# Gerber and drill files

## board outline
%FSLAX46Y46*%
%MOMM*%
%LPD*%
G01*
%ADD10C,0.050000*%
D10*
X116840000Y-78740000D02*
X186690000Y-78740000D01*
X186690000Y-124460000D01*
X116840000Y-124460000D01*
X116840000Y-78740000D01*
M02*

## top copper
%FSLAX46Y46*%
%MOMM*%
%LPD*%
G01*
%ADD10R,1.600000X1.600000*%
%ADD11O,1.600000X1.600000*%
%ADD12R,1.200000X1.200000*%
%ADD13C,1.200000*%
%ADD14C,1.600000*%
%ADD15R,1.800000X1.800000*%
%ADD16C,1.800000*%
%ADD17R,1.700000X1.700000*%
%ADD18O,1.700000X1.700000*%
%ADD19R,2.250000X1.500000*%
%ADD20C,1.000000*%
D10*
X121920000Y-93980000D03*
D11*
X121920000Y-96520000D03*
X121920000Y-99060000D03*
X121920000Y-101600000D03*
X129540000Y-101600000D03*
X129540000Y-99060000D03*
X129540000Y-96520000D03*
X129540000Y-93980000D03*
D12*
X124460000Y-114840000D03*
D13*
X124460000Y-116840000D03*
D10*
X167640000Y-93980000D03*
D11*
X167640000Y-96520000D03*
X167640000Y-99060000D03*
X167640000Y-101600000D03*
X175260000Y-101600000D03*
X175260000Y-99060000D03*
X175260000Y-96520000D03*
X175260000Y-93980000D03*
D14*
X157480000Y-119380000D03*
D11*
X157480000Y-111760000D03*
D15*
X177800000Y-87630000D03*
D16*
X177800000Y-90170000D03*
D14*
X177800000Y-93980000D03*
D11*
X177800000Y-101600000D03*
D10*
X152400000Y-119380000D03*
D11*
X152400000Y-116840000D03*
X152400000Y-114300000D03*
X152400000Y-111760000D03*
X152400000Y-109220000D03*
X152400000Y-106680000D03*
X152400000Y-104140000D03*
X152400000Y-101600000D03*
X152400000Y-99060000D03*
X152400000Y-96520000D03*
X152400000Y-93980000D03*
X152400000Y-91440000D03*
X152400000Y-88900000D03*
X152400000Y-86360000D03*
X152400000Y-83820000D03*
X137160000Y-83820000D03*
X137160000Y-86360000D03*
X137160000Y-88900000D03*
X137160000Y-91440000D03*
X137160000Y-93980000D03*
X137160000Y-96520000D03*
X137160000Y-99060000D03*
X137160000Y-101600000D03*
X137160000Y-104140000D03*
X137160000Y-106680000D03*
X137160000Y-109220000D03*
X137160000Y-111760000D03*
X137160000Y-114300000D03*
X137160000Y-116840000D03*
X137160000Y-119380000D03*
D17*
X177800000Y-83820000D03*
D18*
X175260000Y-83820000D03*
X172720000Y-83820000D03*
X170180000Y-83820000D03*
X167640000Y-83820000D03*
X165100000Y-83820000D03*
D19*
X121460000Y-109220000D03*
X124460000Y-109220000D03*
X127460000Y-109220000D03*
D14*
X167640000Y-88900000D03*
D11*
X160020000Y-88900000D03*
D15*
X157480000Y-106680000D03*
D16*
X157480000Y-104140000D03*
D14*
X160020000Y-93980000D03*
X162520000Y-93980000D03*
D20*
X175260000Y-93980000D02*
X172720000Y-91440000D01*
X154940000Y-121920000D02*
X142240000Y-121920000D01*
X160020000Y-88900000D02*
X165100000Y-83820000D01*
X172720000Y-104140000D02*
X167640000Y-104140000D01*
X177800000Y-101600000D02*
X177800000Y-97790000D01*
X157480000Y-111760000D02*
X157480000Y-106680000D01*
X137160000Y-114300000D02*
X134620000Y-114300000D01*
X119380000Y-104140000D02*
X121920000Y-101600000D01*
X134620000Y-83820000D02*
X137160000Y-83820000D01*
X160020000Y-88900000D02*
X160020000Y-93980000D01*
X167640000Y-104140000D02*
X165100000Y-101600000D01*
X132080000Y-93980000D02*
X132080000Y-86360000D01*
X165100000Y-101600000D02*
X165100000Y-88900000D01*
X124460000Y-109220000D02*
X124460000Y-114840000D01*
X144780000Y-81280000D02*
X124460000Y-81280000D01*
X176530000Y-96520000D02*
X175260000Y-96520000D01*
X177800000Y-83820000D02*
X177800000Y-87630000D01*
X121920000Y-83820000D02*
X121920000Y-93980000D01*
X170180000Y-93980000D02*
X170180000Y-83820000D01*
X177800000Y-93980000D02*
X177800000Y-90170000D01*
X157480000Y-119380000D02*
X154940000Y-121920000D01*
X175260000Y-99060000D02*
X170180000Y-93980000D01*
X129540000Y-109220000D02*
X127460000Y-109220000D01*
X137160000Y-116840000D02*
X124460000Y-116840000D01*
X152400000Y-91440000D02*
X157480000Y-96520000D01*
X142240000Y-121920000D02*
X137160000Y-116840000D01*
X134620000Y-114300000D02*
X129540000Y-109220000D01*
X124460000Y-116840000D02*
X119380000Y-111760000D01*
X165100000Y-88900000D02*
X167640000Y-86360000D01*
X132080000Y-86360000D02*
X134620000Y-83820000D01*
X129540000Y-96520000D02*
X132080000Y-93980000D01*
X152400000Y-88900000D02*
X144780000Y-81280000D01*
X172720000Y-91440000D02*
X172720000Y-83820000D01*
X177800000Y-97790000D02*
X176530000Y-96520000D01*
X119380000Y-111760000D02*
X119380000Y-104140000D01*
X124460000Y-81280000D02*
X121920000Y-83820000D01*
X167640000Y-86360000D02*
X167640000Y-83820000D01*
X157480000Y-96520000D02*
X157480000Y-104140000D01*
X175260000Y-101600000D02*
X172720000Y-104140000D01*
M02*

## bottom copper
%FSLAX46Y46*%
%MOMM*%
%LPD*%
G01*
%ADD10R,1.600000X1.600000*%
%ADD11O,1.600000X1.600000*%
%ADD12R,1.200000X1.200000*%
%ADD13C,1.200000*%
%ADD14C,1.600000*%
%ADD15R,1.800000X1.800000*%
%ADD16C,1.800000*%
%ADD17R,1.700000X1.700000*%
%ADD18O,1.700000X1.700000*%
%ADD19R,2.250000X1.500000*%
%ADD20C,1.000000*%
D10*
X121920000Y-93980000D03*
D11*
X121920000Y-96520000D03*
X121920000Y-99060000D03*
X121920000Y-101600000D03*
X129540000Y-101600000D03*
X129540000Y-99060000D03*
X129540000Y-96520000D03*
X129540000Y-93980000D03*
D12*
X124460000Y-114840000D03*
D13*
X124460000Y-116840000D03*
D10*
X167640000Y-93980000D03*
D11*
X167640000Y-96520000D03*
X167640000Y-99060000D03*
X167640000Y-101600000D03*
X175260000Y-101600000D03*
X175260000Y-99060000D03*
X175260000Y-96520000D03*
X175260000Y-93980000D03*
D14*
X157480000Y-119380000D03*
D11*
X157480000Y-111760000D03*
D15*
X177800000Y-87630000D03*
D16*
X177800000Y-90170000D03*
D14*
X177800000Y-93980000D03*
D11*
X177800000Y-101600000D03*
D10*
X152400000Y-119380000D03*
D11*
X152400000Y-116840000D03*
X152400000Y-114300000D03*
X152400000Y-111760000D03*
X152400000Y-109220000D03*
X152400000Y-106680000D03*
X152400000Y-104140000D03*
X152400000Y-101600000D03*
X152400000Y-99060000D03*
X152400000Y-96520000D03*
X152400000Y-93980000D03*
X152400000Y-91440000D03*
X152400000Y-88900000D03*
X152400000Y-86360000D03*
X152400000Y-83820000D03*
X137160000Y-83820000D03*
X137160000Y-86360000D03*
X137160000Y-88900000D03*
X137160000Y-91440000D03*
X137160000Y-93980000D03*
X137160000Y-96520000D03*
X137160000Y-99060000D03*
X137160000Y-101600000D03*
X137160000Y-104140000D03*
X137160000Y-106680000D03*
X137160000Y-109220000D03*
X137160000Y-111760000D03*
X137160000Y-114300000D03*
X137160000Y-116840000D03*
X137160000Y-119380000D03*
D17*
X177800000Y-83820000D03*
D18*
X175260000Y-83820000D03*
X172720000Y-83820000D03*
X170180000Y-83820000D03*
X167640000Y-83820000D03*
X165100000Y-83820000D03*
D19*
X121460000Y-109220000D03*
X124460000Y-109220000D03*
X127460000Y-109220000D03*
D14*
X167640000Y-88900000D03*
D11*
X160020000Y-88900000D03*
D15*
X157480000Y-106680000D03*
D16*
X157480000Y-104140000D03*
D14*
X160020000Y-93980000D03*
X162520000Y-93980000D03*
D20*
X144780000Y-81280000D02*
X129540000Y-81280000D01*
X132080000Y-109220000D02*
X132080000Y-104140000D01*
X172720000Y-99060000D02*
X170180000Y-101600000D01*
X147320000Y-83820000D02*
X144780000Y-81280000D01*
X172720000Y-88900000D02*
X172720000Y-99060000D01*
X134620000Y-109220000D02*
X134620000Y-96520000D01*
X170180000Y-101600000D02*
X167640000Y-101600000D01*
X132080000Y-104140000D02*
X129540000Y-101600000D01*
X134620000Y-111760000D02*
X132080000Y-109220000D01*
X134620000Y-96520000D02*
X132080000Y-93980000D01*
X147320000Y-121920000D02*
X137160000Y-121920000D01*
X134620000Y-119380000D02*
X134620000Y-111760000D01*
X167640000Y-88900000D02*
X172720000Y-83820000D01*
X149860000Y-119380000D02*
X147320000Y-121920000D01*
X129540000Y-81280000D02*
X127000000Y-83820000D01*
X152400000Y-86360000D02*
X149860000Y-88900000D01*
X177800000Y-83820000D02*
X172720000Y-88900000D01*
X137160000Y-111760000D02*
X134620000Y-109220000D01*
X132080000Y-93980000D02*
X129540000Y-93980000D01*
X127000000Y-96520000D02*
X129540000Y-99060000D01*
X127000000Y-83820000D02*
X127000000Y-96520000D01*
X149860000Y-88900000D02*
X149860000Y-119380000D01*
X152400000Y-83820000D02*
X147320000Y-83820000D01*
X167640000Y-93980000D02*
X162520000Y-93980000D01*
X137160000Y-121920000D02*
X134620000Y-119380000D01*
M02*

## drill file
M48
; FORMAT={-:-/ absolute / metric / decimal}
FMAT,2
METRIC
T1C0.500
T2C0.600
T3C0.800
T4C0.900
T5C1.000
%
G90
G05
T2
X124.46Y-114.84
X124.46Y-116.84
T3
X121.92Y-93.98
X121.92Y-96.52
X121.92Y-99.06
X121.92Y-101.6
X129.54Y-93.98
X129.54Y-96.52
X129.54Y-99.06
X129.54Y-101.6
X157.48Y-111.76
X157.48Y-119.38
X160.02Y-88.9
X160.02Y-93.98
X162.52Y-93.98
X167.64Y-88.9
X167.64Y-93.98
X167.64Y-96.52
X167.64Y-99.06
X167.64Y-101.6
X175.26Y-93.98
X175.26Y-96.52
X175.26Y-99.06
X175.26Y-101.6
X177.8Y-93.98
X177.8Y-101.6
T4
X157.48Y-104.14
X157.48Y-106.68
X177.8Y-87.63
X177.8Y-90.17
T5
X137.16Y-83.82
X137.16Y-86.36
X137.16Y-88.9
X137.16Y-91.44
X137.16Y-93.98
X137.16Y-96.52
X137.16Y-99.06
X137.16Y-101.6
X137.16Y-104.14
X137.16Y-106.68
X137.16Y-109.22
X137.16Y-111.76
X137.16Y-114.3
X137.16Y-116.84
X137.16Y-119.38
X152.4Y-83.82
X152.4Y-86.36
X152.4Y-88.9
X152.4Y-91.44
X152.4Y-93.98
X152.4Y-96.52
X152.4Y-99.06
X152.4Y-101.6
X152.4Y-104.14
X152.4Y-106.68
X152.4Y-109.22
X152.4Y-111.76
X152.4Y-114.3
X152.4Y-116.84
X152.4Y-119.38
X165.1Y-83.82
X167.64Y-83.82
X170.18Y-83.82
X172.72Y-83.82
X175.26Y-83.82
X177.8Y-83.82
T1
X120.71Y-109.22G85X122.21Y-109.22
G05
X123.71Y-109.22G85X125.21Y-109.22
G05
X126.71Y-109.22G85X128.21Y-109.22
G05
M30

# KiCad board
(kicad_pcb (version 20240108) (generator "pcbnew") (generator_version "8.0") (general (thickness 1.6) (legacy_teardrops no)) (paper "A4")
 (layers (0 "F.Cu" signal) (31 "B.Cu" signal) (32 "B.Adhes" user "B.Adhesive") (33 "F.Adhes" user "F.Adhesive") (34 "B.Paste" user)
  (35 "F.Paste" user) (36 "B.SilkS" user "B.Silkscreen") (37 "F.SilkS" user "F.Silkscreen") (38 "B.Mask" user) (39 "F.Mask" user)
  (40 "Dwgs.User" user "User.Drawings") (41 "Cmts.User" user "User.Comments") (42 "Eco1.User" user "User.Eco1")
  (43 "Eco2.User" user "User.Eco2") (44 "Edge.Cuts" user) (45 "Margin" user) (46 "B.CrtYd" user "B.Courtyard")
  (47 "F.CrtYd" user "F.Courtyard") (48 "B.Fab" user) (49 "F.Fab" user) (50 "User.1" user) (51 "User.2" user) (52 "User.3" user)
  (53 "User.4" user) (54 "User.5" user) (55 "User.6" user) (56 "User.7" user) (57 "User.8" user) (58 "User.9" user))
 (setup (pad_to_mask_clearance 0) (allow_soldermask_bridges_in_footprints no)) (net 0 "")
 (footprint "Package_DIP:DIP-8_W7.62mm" (layer "F.Cu") (at 121.92 93.98)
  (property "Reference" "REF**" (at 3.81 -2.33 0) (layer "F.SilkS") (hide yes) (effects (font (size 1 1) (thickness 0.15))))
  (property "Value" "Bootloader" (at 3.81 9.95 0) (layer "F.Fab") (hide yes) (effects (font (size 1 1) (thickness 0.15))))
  (pad "1" thru_hole rect (at 0 0) (size 1.6 1.6) (drill 0.8) (layers "*.Cu" "*.Mask") (remove_unused_layers no))
  (pad "2" thru_hole oval (at 0 2.54) (size 1.6 1.6) (drill 0.8) (layers "*.Cu" "*.Mask") (remove_unused_layers no))
  (pad "3" thru_hole oval (at 0 5.08) (size 1.6 1.6) (drill 0.8) (layers "*.Cu" "*.Mask") (remove_unused_layers no))
  (pad "4" thru_hole oval (at 0 7.62) (size 1.6 1.6) (drill 0.8) (layers "*.Cu" "*.Mask") (remove_unused_layers no))
  (pad "5" thru_hole oval (at 7.62 7.62) (size 1.6 1.6) (drill 0.8) (layers "*.Cu" "*.Mask") (remove_unused_layers no))
  (pad "6" thru_hole oval (at 7.62 5.08) (size 1.6 1.6) (drill 0.8) (layers "*.Cu" "*.Mask") (remove_unused_layers no))
  (pad "7" thru_hole oval (at 7.62 2.54) (size 1.6 1.6) (drill 0.8) (layers "*.Cu" "*.Mask") (remove_unused_layers no))
  (pad "8" thru_hole oval (at 7.62 0) (size 1.6 1.6) (drill 0.8) (layers "*.Cu" "*.Mask") (remove_unused_layers no)))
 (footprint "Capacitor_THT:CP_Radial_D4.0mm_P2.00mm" (layer "F.Cu") (at 124.46 114.84 -90)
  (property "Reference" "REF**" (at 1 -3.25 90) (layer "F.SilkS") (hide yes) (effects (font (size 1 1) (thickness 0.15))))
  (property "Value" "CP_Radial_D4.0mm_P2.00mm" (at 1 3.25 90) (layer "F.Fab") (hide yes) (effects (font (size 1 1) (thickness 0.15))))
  (pad "1" thru_hole rect (at 0 0 270) (size 1.2 1.2) (drill 0.6) (layers "*.Cu" "*.Mask") (remove_unused_layers no))
  (pad "2" thru_hole circle (at 2 0 270) (size 1.2 1.2) (drill 0.6) (layers "*.Cu" "*.Mask") (remove_unused_layers no)))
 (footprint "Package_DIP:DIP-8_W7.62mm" (layer "F.Cu") (at 167.64 93.98)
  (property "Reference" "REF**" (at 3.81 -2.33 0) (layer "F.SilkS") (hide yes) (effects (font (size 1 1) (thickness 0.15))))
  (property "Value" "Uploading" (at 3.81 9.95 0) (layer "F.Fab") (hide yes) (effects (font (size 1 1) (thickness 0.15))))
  (pad "1" thru_hole rect (at 0 0) (size 1.6 1.6) (drill 0.8) (layers "*.Cu" "*.Mask") (remove_unused_layers no))
  (pad "2" thru_hole oval (at 0 2.54) (size 1.6 1.6) (drill 0.8) (layers "*.Cu" "*.Mask") (remove_unused_layers no))
  (pad "3" thru_hole oval (at 0 5.08) (size 1.6 1.6) (drill 0.8) (layers "*.Cu" "*.Mask") (remove_unused_layers no))
  (pad "4" thru_hole oval (at 0 7.62) (size 1.6 1.6) (drill 0.8) (layers "*.Cu" "*.Mask") (remove_unused_layers no))
  (pad "5" thru_hole oval (at 7.62 7.62) (size 1.6 1.6) (drill 0.8) (layers "*.Cu" "*.Mask") (remove_unused_layers no))
  (pad "6" thru_hole oval (at 7.62 5.08) (size 1.6 1.6) (drill 0.8) (layers "*.Cu" "*.Mask") (remove_unused_layers no))
  (pad "7" thru_hole oval (at 7.62 2.54) (size 1.6 1.6) (drill 0.8) (layers "*.Cu" "*.Mask") (remove_unused_layers no))
  (pad "8" thru_hole oval (at 7.62 0) (size 1.6 1.6) (drill 0.8) (layers "*.Cu" "*.Mask") (remove_unused_layers no)))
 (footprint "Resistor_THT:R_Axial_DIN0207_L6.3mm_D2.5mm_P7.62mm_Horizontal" (layer "F.Cu") (at 157.48 119.38 90)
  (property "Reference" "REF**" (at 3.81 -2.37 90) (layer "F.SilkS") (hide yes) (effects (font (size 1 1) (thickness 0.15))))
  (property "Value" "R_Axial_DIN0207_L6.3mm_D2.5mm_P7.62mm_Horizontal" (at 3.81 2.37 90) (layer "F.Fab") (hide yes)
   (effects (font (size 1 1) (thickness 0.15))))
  (pad "1" thru_hole circle (at 0 0 90) (size 1.6 1.6) (drill 0.8) (layers "*.Cu" "*.Mask") (remove_unused_layers no))
  (pad "2" thru_hole oval (at 7.62 0 90) (size 1.6 1.6) (drill 0.8) (layers "*.Cu" "*.Mask") (remove_unused_layers no)))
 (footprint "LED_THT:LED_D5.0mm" (layer "F.Cu") (at 177.8 87.63 -90)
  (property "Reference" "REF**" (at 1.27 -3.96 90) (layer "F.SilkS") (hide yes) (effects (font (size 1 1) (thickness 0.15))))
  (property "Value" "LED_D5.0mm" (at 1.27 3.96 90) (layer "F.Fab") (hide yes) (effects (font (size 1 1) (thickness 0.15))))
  (pad "1" thru_hole rect (at 0 0 270) (size 1.8 1.8) (drill 0.9) (layers "*.Cu" "*.Mask") (remove_unused_layers no))
  (pad "2" thru_hole circle (at 2.54 0 270) (size 1.8 1.8) (drill 0.9) (layers "*.Cu" "*.Mask") (remove_unused_layers no)))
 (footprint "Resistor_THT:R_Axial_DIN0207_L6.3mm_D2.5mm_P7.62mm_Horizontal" (layer "F.Cu") (at 177.8 93.98 -90)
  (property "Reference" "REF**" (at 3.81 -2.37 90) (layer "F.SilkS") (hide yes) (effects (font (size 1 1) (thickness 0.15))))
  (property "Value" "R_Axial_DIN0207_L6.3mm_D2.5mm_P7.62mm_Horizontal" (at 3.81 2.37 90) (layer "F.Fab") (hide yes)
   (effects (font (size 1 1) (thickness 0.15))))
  (pad "1" thru_hole circle (at 0 0 270) (size 1.6 1.6) (drill 0.8) (layers "*.Cu" "*.Mask") (remove_unused_layers no))
  (pad "2" thru_hole oval (at 7.62 0 270) (size 1.6 1.6) (drill 0.8) (layers "*.Cu" "*.Mask") (remove_unused_layers no)))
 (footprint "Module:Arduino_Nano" (layer "F.Cu") (at 152.4 119.38 180)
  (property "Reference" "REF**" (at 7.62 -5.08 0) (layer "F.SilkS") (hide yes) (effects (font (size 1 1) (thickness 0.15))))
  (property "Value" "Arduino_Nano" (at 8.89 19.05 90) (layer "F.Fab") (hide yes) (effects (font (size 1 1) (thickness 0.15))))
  (pad "1" thru_hole rect (at 0 0 180) (size 1.6 1.6) (drill 1) (layers "*.Cu" "*.Mask") (remove_unused_layers no))
  (pad "2" thru_hole oval (at 0 2.54 180) (size 1.6 1.6) (drill 1) (layers "*.Cu" "*.Mask") (remove_unused_layers no))
  (pad "3" thru_hole oval (at 0 5.08 180) (size 1.6 1.6) (drill 1) (layers "*.Cu" "*.Mask") (remove_unused_layers no))
  (pad "4" thru_hole oval (at 0 7.62 180) (size 1.6 1.6) (drill 1) (layers "*.Cu" "*.Mask") (remove_unused_layers no))
  (pad "5" thru_hole oval (at 0 10.16 180) (size 1.6 1.6) (drill 1) (layers "*.Cu" "*.Mask") (remove_unused_layers no))
  (pad "6" thru_hole oval (at 0 12.7 180) (size 1.6 1.6) (drill 1) (layers "*.Cu" "*.Mask") (remove_unused_layers no))
  (pad "7" thru_hole oval (at 0 15.24 180) (size 1.6 1.6) (drill 1) (layers "*.Cu" "*.Mask") (remove_unused_layers no))
  (pad "8" thru_hole oval (at 0 17.78 180) (size 1.6 1.6) (drill 1) (layers "*.Cu" "*.Mask") (remove_unused_layers no))
  (pad "9" thru_hole oval (at 0 20.32 180) (size 1.6 1.6) (drill 1) (layers "*.Cu" "*.Mask") (remove_unused_layers no))
  (pad "10" thru_hole oval (at 0 22.86 180) (size 1.6 1.6) (drill 1) (layers "*.Cu" "*.Mask") (remove_unused_layers no))
  (pad "11" thru_hole oval (at 0 25.4 180) (size 1.6 1.6) (drill 1) (layers "*.Cu" "*.Mask") (remove_unused_layers no))
  (pad "12" thru_hole oval (at 0 27.94 180) (size 1.6 1.6) (drill 1) (layers "*.Cu" "*.Mask") (remove_unused_layers no))
  (pad "13" thru_hole oval (at 0 30.48 180) (size 1.6 1.6) (drill 1) (layers "*.Cu" "*.Mask") (remove_unused_layers no))
  (pad "14" thru_hole oval (at 0 33.02 180) (size 1.6 1.6) (drill 1) (layers "*.Cu" "*.Mask") (remove_unused_layers no))
  (pad "15" thru_hole oval (at 0 35.56 180) (size 1.6 1.6) (drill 1) (layers "*.Cu" "*.Mask") (remove_unused_layers no))
  (pad "16" thru_hole oval (at 15.24 35.56 180) (size 1.6 1.6) (drill 1) (layers "*.Cu" "*.Mask") (remove_unused_layers no))
  (pad "17" thru_hole oval (at 15.24 33.02 180) (size 1.6 1.6) (drill 1) (layers "*.Cu" "*.Mask") (remove_unused_layers no))
  (pad "18" thru_hole oval (at 15.24 30.48 180) (size 1.6 1.6) (drill 1) (layers "*.Cu" "*.Mask") (remove_unused_layers no))
  (pad "19" thru_hole oval (at 15.24 27.94 180) (size 1.6 1.6) (drill 1) (layers "*.Cu" "*.Mask") (remove_unused_layers no))
  (pad "20" thru_hole oval (at 15.24 25.4 180) (size 1.6 1.6) (drill 1) (layers "*.Cu" "*.Mask") (remove_unused_layers no))
  (pad "21" thru_hole oval (at 15.24 22.86 180) (size 1.6 1.6) (drill 1) (layers "*.Cu" "*.Mask") (remove_unused_layers no))
  (pad "22" thru_hole oval (at 15.24 20.32 180) (size 1.6 1.6) (drill 1) (layers "*.Cu" "*.Mask") (remove_unused_layers no))
  (pad "23" thru_hole oval (at 15.24 17.78 180) (size 1.6 1.6) (drill 1) (layers "*.Cu" "*.Mask") (remove_unused_layers no))
  (pad "24" thru_hole oval (at 15.24 15.24 180) (size 1.6 1.6) (drill 1) (layers "*.Cu" "*.Mask") (remove_unused_layers no))
  (pad "25" thru_hole oval (at 15.24 12.7 180) (size 1.6 1.6) (drill 1) (layers "*.Cu" "*.Mask") (remove_unused_layers no))
  (pad "26" thru_hole oval (at 15.24 10.16 180) (size 1.6 1.6) (drill 1) (layers "*.Cu" "*.Mask") (remove_unused_layers no))
  (pad "27" thru_hole oval (at 15.24 7.62 180) (size 1.6 1.6) (drill 1) (layers "*.Cu" "*.Mask") (remove_unused_layers no))
  (pad "28" thru_hole oval (at 15.24 5.08 180) (size 1.6 1.6) (drill 1) (layers "*.Cu" "*.Mask") (remove_unused_layers no))
  (pad "29" thru_hole oval (at 15.24 2.54 180) (size 1.6 1.6) (drill 1) (layers "*.Cu" "*.Mask") (remove_unused_layers no))
  (pad "30" thru_hole oval (at 15.24 0 180) (size 1.6 1.6) (drill 1) (layers "*.Cu" "*.Mask") (remove_unused_layers no)))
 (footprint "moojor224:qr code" (layer "F.Cu") (at 172.72 116.84)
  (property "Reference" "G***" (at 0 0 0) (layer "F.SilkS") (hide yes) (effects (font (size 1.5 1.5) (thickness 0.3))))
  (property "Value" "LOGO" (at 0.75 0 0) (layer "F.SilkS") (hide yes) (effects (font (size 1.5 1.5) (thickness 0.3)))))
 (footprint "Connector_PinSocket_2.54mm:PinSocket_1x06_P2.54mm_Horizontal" (layer "F.Cu") (at 177.8 83.82 -90)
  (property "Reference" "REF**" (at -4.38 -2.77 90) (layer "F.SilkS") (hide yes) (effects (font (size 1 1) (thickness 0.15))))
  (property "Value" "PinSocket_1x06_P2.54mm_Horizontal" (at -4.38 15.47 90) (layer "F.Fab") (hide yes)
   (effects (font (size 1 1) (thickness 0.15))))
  (pad "1" thru_hole rect (at 0 0 270) (size 1.7 1.7) (drill 1) (layers "*.Cu" "*.Mask") (remove_unused_layers no))
  (pad "2" thru_hole oval (at 0 2.54 270) (size 1.7 1.7) (drill 1) (layers "*.Cu" "*.Mask") (remove_unused_layers no))
  (pad "3" thru_hole oval (at 0 5.08 270) (size 1.7 1.7) (drill 1) (layers "*.Cu" "*.Mask") (remove_unused_layers no))
  (pad "4" thru_hole oval (at 0 7.62 270) (size 1.7 1.7) (drill 1) (layers "*.Cu" "*.Mask") (remove_unused_layers no))
  (pad "5" thru_hole oval (at 0 10.16 270) (size 1.7 1.7) (drill 1) (layers "*.Cu" "*.Mask") (remove_unused_layers no))
  (pad "6" thru_hole oval (at 0 12.7 270) (size 1.7 1.7) (drill 1) (layers "*.Cu" "*.Mask") (remove_unused_layers no)))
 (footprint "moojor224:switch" (layer "F.Cu") (at 124.46 109.22)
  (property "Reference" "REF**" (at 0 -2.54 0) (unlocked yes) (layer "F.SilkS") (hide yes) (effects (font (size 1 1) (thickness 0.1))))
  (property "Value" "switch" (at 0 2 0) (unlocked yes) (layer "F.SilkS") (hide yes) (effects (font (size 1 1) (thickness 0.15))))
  (pad "1" thru_hole rect (at -3 0) (size 2.25 1.5) (drill oval 2 0.5) (layers "*.Cu" "*.Mask") (remove_unused_layers no))
  (pad "2" thru_hole rect (at 0 0) (size 2.25 1.5) (drill oval 2 0.5) (layers "*.Cu" "*.Mask") (remove_unused_layers no))
  (pad "3" thru_hole rect (at 3 0) (size 2.25 1.5) (drill oval 2 0.5) (layers "*.Cu" "*.Mask") (remove_unused_layers no)))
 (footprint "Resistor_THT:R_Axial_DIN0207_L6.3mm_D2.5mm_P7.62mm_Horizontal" (layer "F.Cu") (at 167.64 88.9 180)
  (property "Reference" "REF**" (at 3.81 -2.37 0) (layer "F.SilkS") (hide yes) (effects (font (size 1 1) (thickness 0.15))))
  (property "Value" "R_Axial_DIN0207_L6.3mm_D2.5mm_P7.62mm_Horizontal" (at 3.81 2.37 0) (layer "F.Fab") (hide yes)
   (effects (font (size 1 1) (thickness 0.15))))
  (pad "1" thru_hole circle (at 0 0 180) (size 1.6 1.6) (drill 0.8) (layers "*.Cu" "*.Mask") (remove_unused_layers no))
  (pad "2" thru_hole oval (at 7.62 0 180) (size 1.6 1.6) (drill 0.8) (layers "*.Cu" "*.Mask") (remove_unused_layers no)))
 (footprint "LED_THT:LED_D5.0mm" (layer "F.Cu") (at 157.48 106.68 90)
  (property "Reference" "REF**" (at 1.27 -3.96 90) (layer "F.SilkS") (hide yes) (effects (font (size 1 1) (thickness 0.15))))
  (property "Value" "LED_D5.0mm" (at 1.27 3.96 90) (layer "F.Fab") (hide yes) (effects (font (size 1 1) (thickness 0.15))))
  (pad "1" thru_hole rect (at 0 0 90) (size 1.8 1.8) (drill 0.9) (layers "*.Cu" "*.Mask") (remove_unused_layers no))
  (pad "2" thru_hole circle (at 2.54 0 90) (size 1.8 1.8) (drill 0.9) (layers "*.Cu" "*.Mask") (remove_unused_layers no)))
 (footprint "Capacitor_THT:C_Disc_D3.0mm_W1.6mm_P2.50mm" (layer "F.Cu") (at 160.02 93.98)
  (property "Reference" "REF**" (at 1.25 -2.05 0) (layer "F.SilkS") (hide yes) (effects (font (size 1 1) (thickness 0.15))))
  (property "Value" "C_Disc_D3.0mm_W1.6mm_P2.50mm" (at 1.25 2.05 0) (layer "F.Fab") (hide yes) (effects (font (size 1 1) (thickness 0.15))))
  (pad "1" thru_hole circle (at 0 0) (size 1.6 1.6) (drill 0.8) (layers "*.Cu" "*.Mask") (remove_unused_layers no))
  (pad "2" thru_hole circle (at 2.5 0) (size 1.6 1.6) (drill 0.8) (layers "*.Cu" "*.Mask") (remove_unused_layers no)))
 (gr_rect (start 116.84 78.74) (end 186.69 124.46) (stroke (width 0.05) (type default)) (fill none) (layer "Edge.Cuts"))
 (segment (start 175.26 93.98) (end 172.72 91.44) (width 1) (layer "F.Cu") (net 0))
 (segment (start 154.94 121.92) (end 142.24 121.92) (width 1) (layer "F.Cu") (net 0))
 (segment (start 160.02 88.9) (end 165.1 83.82) (width 1) (layer "F.Cu") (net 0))
 (segment (start 172.72 104.14) (end 167.64 104.14) (width 1) (layer "F.Cu") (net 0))
 (segment (start 177.8 101.6) (end 177.8 97.79) (width 1) (layer "F.Cu") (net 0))
 (segment (start 157.48 111.76) (end 157.48 106.68) (width 1) (layer "F.Cu") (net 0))
 (segment (start 137.16 114.3) (end 134.62 114.3) (width 1) (layer "F.Cu") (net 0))
 (segment (start 119.38 104.14) (end 121.92 101.6) (width 1) (layer "F.Cu") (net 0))
 (segment (start 134.62 83.82) (end 137.16 83.82) (width 1) (layer "F.Cu") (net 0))
 (segment (start 160.02 88.9) (end 160.02 93.98) (width 1) (layer "F.Cu") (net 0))
 (segment (start 167.64 104.14) (end 165.1 101.6) (width 1) (layer "F.Cu") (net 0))
 (segment (start 132.08 93.98) (end 132.08 86.36) (width 1) (layer "F.Cu") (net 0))
 (segment (start 165.1 101.6) (end 165.1 88.9) (width 1) (layer "F.Cu") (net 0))
 (segment (start 124.46 109.22) (end 124.46 114.84) (width 1) (layer "F.Cu") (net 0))
 (segment (start 144.78 81.28) (end 124.46 81.28) (width 1) (layer "F.Cu") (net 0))
 (segment (start 176.53 96.52) (end 175.26 96.52) (width 1) (layer "F.Cu") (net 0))
 (segment (start 177.8 83.82) (end 177.8 87.63) (width 1) (layer "F.Cu") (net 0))
 (segment (start 121.92 83.82) (end 121.92 93.98) (width 1) (layer "F.Cu") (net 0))
 (segment (start 170.18 93.98) (end 170.18 83.82) (width 1) (layer "F.Cu") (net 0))
 (segment (start 177.8 93.98) (end 177.8 90.17) (width 1) (layer "F.Cu") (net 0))
 (segment (start 157.48 119.38) (end 154.94 121.92) (width 1) (layer "F.Cu") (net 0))
 (segment (start 175.26 99.06) (end 170.18 93.98) (width 1) (layer "F.Cu") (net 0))
 (segment (start 129.54 109.22) (end 127.46 109.22) (width 1) (layer "F.Cu") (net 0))
 (segment (start 137.16 116.84) (end 124.46 116.84) (width 1) (layer "F.Cu") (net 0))
 (segment (start 152.4 91.44) (end 157.48 96.52) (width 1) (layer "F.Cu") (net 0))
 (segment (start 142.24 121.92) (end 137.16 116.84) (width 1) (layer "F.Cu") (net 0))
 (segment (start 134.62 114.3) (end 129.54 109.22) (width 1) (layer "F.Cu") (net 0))
 (segment (start 124.46 116.84) (end 119.38 111.76) (width 1) (layer "F.Cu") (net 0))
 (segment (start 165.1 88.9) (end 167.64 86.36) (width 1) (layer "F.Cu") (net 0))
 (segment (start 132.08 86.36) (end 134.62 83.82) (width 1) (layer "F.Cu") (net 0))
 (segment (start 129.54 96.52) (end 132.08 93.98) (width 1) (layer "F.Cu") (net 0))
 (segment (start 152.4 88.9) (end 144.78 81.28) (width 1) (layer "F.Cu") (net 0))
 (segment (start 172.72 91.44) (end 172.72 83.82) (width 1) (layer "F.Cu") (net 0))
 (segment (start 177.8 97.79) (end 176.53 96.52) (width 1) (layer "F.Cu") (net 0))
 (segment (start 119.38 111.76) (end 119.38 104.14) (width 1) (layer "F.Cu") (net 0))
 (segment (start 124.46 81.28) (end 121.92 83.82) (width 1) (layer "F.Cu") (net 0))
 (segment (start 167.64 86.36) (end 167.64 83.82) (width 1) (layer "F.Cu") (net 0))
 (segment (start 157.48 96.52) (end 157.48 104.14) (width 1) (layer "F.Cu") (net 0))
 (segment (start 175.26 101.6) (end 172.72 104.14) (width 1) (layer "F.Cu") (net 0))
 (segment (start 144.78 81.28) (end 129.54 81.28) (width 1) (layer "B.Cu") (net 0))
 (segment (start 132.08 109.22) (end 132.08 104.14) (width 1) (layer "B.Cu") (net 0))
 (segment (start 172.72 99.06) (end 170.18 101.6) (width 1) (layer "B.Cu") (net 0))
 (segment (start 147.32 83.82) (end 144.78 81.28) (width 1) (layer "B.Cu") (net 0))
 (segment (start 172.72 88.9) (end 172.72 99.06) (width 1) (layer "B.Cu") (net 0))
 (segment (start 134.62 109.22) (end 134.62 96.52) (width 1) (layer "B.Cu") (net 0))
 (segment (start 170.18 101.6) (end 167.64 101.6) (width 1) (layer "B.Cu") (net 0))
 (segment (start 132.08 104.14) (end 129.54 101.6) (width 1) (layer "B.Cu") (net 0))
 (segment (start 134.62 111.76) (end 132.08 109.22) (width 1) (layer "B.Cu") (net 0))
 (segment (start 134.62 96.52) (end 132.08 93.98) (width 1) (layer "B.Cu") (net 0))
 (segment (start 147.32 121.92) (end 137.16 121.92) (width 1) (layer "B.Cu") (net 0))
 (segment (start 134.62 119.38) (end 134.62 111.76) (width 1) (layer "B.Cu") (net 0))
 (segment (start 167.64 88.9) (end 172.72 83.82) (width 1) (layer "B.Cu") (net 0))
 (segment (start 149.86 119.38) (end 147.32 121.92) (width 1) (layer "B.Cu") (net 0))
 (segment (start 129.54 81.28) (end 127 83.82) (width 1) (layer "B.Cu") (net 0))
 (segment (start 152.4 86.36) (end 149.86 88.9) (width 1) (layer "B.Cu") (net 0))
 (segment (start 177.8 83.82) (end 172.72 88.9) (width 1) (layer "B.Cu") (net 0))
 (segment (start 137.16 111.76) (end 134.62 109.22) (width 1) (layer "B.Cu") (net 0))
 (segment (start 132.08 93.98) (end 129.54 93.98) (width 1) (layer "B.Cu") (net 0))
 (segment (start 127 96.52) (end 129.54 99.06) (width 1) (layer "B.Cu") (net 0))
 (segment (start 127 83.82) (end 127 96.52) (width 1) (layer "B.Cu") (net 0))
 (segment (start 149.86 88.9) (end 149.86 119.38) (width 1) (layer "B.Cu") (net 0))
 (segment (start 152.4 83.82) (end 147.32 83.82) (width 1) (layer "B.Cu") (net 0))
 (segment (start 167.64 93.98) (end 162.52 93.98) (width 1) (layer "B.Cu") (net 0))
 (segment (start 137.16 121.92) (end 134.62 119.38) (width 1) (layer "B.Cu") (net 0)))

